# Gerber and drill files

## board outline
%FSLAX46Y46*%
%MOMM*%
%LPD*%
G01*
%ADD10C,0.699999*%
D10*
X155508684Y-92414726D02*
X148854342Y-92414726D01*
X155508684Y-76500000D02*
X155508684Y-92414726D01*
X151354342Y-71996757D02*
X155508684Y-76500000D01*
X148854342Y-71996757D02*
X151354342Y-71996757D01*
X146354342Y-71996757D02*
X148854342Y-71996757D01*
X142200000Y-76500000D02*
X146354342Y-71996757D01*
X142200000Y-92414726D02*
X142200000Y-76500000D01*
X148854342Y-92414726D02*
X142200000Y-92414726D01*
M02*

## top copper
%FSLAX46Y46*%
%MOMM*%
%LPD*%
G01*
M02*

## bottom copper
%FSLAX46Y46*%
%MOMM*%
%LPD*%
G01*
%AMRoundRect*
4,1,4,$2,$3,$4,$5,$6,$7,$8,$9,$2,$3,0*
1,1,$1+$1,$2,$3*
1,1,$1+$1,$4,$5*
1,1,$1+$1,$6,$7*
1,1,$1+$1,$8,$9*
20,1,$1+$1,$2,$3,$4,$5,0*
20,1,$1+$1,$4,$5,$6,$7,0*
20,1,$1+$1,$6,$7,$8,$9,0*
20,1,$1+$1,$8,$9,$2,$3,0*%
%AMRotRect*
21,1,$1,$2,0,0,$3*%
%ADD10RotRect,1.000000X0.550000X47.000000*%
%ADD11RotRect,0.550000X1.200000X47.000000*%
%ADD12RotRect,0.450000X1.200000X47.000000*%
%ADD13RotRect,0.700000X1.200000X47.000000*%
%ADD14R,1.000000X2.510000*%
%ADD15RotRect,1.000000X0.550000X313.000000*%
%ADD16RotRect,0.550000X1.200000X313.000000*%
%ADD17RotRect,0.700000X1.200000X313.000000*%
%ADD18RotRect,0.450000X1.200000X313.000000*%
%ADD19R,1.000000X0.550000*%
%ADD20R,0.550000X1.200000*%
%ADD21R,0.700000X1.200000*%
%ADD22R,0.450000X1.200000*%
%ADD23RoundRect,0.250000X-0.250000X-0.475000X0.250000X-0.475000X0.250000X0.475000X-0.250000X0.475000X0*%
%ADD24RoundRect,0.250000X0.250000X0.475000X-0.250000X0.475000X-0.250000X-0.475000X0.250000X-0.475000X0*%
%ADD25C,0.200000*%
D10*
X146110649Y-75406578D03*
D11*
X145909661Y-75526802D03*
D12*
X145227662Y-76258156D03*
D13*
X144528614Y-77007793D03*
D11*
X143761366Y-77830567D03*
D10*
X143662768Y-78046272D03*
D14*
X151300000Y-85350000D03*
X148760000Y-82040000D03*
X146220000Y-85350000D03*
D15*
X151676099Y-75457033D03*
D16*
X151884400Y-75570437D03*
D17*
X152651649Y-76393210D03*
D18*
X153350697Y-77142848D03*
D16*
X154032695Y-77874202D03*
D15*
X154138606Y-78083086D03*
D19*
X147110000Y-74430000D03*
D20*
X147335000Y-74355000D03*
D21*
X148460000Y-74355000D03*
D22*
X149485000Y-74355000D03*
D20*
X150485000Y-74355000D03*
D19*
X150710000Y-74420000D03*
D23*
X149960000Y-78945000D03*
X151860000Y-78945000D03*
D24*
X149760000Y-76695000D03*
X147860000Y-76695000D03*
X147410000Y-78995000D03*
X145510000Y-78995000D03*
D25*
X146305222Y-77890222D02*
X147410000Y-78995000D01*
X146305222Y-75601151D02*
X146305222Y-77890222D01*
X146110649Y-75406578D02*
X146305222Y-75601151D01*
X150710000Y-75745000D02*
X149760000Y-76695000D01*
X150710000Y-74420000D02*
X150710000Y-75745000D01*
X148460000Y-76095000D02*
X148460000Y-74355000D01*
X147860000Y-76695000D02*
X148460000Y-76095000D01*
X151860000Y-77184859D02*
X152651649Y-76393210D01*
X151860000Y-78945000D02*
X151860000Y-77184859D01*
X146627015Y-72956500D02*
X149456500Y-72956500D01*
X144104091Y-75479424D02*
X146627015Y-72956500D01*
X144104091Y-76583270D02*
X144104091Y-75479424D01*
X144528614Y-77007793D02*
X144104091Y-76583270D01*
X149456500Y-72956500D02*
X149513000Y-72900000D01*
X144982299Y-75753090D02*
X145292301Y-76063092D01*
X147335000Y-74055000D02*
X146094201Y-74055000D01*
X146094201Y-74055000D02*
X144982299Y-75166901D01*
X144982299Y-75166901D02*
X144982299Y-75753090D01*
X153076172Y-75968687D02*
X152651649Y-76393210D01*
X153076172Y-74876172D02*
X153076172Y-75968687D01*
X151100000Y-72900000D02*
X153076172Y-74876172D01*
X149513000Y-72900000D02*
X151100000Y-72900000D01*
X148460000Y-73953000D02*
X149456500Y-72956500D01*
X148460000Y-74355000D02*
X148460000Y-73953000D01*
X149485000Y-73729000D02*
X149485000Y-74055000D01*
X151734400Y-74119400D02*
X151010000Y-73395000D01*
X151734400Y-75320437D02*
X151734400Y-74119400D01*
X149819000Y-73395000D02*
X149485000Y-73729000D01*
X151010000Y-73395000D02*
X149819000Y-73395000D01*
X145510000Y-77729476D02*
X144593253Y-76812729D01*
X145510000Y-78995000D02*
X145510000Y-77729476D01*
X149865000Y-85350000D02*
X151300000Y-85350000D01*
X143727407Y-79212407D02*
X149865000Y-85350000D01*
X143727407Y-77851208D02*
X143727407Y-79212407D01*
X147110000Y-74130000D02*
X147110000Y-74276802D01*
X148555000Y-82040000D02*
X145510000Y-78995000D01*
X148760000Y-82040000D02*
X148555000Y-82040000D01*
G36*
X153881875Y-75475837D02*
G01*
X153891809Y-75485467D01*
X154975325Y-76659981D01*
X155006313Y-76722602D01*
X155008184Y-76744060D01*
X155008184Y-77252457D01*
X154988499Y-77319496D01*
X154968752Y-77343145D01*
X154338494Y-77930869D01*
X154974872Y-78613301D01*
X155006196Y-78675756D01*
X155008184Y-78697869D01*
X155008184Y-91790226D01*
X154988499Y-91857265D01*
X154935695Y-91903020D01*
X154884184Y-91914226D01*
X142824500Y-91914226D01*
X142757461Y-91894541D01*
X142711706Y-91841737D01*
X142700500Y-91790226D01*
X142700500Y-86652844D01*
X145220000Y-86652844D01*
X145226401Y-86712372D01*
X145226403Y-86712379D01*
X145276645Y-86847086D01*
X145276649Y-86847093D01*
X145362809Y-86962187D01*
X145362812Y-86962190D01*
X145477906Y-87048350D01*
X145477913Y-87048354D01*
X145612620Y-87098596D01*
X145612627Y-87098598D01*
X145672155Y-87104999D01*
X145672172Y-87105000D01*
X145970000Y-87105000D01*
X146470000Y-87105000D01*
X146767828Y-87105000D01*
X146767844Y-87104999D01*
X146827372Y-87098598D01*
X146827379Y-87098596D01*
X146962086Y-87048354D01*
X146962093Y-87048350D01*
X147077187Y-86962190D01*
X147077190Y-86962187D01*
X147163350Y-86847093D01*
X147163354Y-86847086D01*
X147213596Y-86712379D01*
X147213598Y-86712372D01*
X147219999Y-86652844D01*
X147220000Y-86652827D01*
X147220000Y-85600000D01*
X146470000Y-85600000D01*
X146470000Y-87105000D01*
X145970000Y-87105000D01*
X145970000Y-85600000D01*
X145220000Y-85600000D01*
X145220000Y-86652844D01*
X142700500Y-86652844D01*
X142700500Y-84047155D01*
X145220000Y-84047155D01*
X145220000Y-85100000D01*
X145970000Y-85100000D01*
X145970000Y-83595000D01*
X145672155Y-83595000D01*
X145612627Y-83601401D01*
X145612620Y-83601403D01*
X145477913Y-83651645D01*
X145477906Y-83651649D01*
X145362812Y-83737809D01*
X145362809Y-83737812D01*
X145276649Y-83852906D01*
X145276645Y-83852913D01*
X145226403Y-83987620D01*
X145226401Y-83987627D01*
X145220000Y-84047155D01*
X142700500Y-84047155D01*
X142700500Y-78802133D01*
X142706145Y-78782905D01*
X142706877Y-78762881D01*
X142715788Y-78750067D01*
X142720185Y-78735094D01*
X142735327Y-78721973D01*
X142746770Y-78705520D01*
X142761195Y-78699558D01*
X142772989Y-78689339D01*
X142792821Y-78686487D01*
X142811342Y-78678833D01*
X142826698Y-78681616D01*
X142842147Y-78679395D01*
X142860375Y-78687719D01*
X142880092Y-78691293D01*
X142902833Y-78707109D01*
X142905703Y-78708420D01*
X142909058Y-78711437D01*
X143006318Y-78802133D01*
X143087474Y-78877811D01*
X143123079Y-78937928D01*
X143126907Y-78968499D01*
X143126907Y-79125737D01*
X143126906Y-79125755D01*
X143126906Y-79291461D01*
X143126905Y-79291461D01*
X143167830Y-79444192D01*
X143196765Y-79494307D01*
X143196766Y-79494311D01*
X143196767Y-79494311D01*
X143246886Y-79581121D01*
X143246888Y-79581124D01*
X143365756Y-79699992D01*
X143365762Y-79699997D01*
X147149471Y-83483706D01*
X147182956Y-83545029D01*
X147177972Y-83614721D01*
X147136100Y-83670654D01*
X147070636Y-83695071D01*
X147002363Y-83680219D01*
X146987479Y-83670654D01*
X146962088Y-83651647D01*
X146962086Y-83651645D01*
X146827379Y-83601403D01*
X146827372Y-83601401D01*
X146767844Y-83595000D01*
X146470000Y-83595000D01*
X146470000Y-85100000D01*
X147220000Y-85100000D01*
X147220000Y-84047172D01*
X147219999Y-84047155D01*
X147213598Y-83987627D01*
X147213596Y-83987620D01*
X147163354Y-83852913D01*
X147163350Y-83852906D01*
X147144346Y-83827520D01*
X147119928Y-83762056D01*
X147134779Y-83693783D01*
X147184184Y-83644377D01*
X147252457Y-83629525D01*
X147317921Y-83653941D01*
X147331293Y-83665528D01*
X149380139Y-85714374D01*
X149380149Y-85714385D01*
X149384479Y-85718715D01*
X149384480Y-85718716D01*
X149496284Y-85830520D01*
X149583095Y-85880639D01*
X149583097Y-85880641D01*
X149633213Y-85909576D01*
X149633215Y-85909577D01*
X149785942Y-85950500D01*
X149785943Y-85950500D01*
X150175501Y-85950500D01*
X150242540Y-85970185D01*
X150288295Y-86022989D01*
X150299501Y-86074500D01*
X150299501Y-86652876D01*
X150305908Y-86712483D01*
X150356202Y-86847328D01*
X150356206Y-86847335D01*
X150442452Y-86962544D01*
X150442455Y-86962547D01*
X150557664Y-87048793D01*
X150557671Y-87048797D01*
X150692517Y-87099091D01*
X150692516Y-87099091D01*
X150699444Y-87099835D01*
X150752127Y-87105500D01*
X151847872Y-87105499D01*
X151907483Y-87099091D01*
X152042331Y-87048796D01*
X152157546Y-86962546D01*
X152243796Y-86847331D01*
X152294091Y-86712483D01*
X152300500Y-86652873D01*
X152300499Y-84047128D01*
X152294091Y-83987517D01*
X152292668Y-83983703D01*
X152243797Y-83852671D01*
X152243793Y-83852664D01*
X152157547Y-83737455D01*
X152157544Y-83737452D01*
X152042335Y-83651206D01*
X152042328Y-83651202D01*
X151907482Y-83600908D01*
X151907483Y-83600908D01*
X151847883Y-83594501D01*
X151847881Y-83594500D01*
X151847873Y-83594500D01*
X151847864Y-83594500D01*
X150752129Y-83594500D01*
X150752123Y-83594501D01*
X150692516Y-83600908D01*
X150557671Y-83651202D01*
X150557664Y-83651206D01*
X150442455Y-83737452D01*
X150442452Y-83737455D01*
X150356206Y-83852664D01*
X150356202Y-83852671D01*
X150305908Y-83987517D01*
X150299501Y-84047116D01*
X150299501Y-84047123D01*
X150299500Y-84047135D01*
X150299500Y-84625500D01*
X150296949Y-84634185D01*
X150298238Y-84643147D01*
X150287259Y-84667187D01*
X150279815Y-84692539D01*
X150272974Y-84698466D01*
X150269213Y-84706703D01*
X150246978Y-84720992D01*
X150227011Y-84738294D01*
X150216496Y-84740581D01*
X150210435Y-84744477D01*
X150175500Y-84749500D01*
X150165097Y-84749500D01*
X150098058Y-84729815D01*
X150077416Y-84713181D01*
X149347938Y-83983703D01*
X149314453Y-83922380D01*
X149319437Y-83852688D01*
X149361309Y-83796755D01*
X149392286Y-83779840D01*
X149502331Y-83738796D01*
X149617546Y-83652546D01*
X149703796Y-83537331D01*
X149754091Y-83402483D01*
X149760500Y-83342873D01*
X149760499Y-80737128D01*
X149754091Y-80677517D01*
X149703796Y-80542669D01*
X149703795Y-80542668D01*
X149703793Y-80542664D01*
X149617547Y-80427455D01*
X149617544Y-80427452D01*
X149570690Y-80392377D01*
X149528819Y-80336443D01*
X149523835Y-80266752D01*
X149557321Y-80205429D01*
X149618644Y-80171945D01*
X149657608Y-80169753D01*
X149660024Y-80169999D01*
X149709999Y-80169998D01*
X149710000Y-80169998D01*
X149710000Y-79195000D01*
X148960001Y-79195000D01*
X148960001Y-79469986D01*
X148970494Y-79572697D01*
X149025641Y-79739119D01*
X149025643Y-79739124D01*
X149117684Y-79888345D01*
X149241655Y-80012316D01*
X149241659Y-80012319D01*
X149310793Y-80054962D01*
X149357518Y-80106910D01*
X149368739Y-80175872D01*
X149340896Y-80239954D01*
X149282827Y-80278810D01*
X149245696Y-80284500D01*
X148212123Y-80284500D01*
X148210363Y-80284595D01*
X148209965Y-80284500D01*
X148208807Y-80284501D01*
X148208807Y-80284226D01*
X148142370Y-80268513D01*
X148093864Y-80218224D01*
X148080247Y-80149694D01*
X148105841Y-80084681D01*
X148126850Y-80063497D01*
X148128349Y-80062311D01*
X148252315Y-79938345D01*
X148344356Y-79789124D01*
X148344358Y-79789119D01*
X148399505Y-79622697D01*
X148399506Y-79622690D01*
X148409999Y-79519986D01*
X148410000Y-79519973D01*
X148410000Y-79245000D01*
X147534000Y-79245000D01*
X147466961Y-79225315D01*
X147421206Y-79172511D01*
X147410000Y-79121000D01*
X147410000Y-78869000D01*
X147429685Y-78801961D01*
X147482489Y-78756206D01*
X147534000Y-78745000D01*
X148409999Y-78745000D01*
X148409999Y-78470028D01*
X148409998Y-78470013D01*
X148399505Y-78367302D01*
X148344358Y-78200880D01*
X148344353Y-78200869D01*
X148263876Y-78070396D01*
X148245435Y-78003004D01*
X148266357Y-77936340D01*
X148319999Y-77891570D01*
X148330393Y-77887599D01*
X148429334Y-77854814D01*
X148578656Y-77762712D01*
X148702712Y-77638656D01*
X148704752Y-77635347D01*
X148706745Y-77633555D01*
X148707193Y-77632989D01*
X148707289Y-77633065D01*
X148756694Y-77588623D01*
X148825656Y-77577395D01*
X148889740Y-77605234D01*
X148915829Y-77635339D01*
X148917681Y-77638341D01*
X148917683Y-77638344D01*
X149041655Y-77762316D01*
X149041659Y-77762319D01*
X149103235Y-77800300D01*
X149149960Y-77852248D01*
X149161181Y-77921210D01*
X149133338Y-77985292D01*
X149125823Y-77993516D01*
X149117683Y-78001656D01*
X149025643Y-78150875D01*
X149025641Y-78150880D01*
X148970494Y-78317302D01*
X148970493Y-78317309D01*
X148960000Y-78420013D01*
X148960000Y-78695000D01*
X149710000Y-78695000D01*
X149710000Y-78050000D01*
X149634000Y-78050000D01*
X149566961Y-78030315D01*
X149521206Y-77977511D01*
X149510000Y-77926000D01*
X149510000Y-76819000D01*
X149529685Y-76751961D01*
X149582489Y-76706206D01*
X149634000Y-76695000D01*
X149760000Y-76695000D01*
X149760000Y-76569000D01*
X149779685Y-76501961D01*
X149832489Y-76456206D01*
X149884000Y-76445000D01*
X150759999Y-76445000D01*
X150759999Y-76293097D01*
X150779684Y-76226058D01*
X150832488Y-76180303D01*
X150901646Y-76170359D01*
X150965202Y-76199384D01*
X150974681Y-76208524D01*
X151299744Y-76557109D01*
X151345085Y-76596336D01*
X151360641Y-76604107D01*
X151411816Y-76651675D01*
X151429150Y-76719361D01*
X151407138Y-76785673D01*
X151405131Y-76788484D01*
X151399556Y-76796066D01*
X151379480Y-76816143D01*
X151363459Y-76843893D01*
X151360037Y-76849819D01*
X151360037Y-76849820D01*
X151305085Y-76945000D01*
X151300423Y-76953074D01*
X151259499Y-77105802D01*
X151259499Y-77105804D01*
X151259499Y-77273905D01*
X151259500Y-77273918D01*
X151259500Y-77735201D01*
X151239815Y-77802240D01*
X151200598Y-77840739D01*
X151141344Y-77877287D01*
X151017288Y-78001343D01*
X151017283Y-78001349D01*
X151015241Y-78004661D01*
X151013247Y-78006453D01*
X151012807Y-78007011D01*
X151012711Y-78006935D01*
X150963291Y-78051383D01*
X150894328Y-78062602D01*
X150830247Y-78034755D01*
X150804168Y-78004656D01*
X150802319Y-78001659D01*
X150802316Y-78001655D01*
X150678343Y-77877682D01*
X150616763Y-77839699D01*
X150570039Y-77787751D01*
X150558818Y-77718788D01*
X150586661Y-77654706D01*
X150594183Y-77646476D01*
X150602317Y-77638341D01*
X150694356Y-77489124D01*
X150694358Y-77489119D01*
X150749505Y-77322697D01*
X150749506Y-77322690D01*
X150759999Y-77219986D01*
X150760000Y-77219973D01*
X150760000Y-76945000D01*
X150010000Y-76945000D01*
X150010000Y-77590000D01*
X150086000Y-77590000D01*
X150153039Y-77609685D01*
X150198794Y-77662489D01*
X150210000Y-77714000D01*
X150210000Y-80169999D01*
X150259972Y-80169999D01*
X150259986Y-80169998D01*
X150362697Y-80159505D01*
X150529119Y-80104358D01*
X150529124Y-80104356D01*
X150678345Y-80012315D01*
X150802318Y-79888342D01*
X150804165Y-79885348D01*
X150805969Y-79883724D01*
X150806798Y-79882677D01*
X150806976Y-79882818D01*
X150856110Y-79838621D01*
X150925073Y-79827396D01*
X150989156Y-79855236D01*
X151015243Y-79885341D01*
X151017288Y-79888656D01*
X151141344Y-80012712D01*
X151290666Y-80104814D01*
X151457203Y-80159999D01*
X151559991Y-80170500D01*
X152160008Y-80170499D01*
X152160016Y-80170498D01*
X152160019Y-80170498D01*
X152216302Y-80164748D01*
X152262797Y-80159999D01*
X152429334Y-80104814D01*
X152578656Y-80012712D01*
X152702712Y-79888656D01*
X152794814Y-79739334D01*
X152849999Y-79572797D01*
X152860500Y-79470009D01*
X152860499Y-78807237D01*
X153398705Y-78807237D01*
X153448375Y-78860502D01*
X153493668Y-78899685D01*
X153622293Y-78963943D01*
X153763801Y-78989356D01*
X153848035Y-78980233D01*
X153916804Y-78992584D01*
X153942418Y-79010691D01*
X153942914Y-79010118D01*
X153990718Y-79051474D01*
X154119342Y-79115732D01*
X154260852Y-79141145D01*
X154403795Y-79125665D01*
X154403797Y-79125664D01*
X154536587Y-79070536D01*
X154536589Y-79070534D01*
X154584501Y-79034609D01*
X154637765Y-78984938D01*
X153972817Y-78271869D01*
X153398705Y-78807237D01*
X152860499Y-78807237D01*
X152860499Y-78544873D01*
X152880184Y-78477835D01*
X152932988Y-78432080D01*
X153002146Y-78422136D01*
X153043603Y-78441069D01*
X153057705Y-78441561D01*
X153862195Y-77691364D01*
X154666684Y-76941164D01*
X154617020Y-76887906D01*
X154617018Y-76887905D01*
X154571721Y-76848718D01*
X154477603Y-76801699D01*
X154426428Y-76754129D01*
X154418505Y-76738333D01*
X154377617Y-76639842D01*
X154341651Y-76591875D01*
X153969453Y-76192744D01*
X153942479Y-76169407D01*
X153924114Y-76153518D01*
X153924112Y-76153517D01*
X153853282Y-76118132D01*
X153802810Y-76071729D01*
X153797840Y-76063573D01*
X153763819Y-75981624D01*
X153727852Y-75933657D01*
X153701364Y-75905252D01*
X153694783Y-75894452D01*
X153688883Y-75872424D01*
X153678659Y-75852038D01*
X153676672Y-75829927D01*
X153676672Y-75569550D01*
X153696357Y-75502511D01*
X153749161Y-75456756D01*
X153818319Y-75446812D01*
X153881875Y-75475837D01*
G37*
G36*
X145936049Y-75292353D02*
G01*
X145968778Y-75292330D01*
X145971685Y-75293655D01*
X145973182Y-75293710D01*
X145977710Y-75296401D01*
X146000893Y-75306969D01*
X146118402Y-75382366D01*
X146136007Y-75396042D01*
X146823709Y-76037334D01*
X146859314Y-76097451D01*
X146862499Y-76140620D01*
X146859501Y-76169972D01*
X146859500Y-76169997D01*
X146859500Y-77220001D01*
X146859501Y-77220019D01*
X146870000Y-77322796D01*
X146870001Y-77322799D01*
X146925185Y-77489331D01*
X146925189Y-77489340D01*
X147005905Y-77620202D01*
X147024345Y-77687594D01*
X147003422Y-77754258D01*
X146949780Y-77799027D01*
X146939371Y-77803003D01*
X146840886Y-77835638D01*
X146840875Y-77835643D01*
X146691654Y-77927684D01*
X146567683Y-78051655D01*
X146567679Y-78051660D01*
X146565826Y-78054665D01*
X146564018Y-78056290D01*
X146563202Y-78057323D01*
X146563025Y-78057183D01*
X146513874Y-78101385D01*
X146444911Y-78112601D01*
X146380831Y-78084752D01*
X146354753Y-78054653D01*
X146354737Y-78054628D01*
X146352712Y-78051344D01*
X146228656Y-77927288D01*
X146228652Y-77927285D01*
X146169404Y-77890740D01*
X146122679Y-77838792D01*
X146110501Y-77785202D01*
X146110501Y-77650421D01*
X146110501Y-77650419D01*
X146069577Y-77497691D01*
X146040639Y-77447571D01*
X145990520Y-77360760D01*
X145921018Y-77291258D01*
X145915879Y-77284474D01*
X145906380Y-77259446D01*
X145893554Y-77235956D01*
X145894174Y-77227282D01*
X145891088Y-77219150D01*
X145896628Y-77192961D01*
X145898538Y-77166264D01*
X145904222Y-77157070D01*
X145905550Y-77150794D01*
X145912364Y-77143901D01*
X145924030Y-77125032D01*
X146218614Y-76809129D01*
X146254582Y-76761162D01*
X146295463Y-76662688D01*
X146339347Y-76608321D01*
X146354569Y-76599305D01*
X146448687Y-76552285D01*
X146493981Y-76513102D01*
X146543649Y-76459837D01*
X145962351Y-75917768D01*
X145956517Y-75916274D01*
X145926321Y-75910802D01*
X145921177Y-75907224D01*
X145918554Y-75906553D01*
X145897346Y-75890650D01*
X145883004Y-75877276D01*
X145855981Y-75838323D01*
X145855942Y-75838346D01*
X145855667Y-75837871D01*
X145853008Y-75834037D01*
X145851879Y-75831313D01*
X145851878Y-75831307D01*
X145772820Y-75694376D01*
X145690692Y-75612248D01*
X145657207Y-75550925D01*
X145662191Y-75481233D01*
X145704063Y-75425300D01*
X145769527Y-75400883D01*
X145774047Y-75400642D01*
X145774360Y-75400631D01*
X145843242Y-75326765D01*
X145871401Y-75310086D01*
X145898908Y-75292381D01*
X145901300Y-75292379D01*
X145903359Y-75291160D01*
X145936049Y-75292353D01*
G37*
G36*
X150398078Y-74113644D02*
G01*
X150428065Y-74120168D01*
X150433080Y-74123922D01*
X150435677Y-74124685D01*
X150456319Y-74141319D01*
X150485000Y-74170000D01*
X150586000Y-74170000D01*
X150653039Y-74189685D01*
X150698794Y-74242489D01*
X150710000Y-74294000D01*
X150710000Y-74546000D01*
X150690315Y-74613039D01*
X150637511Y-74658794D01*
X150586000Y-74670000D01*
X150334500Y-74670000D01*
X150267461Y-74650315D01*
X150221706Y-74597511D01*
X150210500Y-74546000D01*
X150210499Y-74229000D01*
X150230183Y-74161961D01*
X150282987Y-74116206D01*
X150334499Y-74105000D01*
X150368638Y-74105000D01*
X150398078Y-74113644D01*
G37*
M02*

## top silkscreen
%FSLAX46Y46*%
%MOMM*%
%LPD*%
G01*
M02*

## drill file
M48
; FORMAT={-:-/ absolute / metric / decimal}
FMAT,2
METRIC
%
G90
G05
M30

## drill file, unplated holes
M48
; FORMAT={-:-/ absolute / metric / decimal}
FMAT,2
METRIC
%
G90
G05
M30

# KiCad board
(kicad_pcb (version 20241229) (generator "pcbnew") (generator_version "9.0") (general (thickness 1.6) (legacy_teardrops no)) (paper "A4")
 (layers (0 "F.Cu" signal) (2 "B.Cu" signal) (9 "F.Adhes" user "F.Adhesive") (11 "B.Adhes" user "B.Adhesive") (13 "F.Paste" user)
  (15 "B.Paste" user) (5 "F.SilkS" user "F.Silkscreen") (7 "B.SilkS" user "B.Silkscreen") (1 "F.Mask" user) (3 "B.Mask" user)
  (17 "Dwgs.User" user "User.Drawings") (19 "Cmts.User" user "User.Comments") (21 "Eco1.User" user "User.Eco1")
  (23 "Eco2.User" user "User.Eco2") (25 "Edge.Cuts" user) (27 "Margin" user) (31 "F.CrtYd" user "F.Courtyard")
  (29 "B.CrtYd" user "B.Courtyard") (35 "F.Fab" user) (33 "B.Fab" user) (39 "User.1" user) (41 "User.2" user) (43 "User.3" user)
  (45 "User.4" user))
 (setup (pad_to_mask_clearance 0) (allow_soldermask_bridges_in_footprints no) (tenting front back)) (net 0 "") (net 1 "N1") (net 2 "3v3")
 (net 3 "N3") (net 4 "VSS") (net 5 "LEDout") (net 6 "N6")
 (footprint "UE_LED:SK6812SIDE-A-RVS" (layer "B.Cu") (at 152.897661 76.642364 -47)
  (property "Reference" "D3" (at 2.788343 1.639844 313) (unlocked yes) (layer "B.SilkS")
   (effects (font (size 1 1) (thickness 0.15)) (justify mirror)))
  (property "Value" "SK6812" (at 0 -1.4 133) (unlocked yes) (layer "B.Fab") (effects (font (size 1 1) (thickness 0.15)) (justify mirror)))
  (pad "1" smd rect (at -1.699999 0.085 313) (size 1 0.55) (layers "B.Cu" "B.Mask" "B.Paste") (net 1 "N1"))
  (pad "1" smd rect (at -1.475 0.01 313) (size 0.55 1.2) (layers "B.Cu" "B.Mask" "B.Paste") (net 1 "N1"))
  (pad "2" smd rect (at -0.349999 0.009999 313) (size 0.7 1.2) (layers "B.Cu" "B.Mask" "B.Paste") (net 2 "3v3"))
  (pad "3" smd rect (at 0.675001 0.01 313) (size 0.45 1.2) (layers "B.Cu" "B.Mask" "B.Paste") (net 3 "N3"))
  (pad "4" smd rect (at 1.675001 0.01 313) (size 0.55 1.2) (layers "B.Cu" "B.Mask" "B.Paste") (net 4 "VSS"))
  (pad "4" smd rect (at 1.9 0.075 313) (size 1 0.55) (layers "B.Cu" "B.Mask" "B.Paste") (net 4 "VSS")))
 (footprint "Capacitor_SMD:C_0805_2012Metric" (layer "B.Cu") (at 150.91 78.945)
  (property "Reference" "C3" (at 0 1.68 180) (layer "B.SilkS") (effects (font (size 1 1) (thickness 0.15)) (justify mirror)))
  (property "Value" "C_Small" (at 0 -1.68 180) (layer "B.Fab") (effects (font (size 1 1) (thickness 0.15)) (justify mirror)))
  (pad "1" smd roundrect (at -0.95 0) (size 1 1.45) (layers "B.Cu" "B.Mask" "B.Paste") (roundrect_rratio 0.25) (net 4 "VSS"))
  (pad "2" smd roundrect (at 0.95 0) (size 1 1.45) (layers "B.Cu" "B.Mask" "B.Paste") (roundrect_rratio 0.25) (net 2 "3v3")))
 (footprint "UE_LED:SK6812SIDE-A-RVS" (layer "B.Cu") (at 144.76 76.745 47)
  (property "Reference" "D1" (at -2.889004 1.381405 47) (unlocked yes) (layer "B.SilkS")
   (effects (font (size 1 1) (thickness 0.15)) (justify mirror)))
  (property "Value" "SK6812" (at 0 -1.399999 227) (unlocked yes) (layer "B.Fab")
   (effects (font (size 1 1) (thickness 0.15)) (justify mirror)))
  (pad "1" smd rect (at -1.700001 0.085001 47) (size 1 0.55) (layers "B.Cu" "B.Mask" "B.Paste") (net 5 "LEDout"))
  (pad "1" smd rect (at -1.475 0.01 47) (size 0.55 1.2) (layers "B.Cu" "B.Mask" "B.Paste") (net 5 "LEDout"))
  (pad "2" smd rect (at -0.35 0.009999 47) (size 0.7 1.2) (layers "B.Cu" "B.Mask" "B.Paste") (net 2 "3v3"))
  (pad "3" smd rect (at 0.675 0.01 47) (size 0.45 1.2) (layers "B.Cu" "B.Mask" "B.Paste") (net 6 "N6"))
  (pad "4" smd rect (at 1.675001 0.01 47) (size 0.55 1.2) (layers "B.Cu" "B.Mask" "B.Paste") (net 4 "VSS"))
  (pad "4" smd rect (at 1.9 0.075001 47) (size 1 0.55) (layers "B.Cu" "B.Mask" "B.Paste") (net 4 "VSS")))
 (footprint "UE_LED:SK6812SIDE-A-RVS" (layer "B.Cu") (at 148.81 74.345)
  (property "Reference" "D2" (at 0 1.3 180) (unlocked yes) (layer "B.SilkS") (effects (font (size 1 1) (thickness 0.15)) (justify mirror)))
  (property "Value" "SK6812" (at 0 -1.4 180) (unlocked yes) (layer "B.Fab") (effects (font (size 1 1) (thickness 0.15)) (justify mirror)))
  (pad "1" smd rect (at -1.7 0.085) (size 1 0.55) (layers "B.Cu" "B.Mask" "B.Paste") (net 6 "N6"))
  (pad "1" smd rect (at -1.475 0.01) (size 0.55 1.2) (layers "B.Cu" "B.Mask" "B.Paste") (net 6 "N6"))
  (pad "2" smd rect (at -0.35 0.01) (size 0.7 1.2) (layers "B.Cu" "B.Mask" "B.Paste") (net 2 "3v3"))
  (pad "3" smd rect (at 0.675 0.01) (size 0.45 1.2) (layers "B.Cu" "B.Mask" "B.Paste") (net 1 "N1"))
  (pad "4" smd rect (at 1.675 0.01) (size 0.55 1.2) (layers "B.Cu" "B.Mask" "B.Paste") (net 4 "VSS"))
  (pad "4" smd rect (at 1.9 0.075) (size 1 0.55) (layers "B.Cu" "B.Mask" "B.Paste") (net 4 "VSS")))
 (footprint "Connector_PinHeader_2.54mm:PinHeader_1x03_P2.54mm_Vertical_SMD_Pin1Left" (layer "B.Cu") (at 148.76 83.695 90)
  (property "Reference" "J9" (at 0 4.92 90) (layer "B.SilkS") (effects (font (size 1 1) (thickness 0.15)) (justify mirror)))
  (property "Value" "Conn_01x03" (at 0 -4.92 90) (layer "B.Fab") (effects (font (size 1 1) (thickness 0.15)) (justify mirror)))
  (pad "1" smd rect (at -1.655 2.54 90) (size 2.51 1) (layers "B.Cu" "B.Mask" "B.Paste") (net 5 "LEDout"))
  (pad "2" smd rect (at 1.655 0 90) (size 2.51 1) (layers "B.Cu" "B.Mask" "B.Paste") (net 2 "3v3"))
  (pad "3" smd rect (at -1.655 -2.54 90) (size 2.51 1) (layers "B.Cu" "B.Mask" "B.Paste") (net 4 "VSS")))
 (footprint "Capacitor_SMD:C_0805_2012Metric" (layer "B.Cu") (at 148.81 76.695 180)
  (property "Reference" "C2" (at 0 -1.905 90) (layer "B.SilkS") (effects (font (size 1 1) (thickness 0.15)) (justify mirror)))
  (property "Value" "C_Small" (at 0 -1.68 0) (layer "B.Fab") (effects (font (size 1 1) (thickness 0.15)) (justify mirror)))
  (pad "1" smd roundrect (at -0.95 0 180) (size 1 1.45) (layers "B.Cu" "B.Mask" "B.Paste") (roundrect_rratio 0.25) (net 4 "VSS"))
  (pad "2" smd roundrect (at 0.95 0 180) (size 1 1.45) (layers "B.Cu" "B.Mask" "B.Paste") (roundrect_rratio 0.25) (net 2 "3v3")))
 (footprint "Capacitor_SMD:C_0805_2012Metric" (layer "B.Cu") (at 146.46 78.995 180)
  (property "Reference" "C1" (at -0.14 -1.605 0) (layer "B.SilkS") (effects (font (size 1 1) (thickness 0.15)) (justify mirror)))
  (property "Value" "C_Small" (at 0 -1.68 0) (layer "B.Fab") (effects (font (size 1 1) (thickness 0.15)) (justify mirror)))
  (pad "1" smd roundrect (at -0.95 0 180) (size 1 1.45) (layers "B.Cu" "B.Mask" "B.Paste") (roundrect_rratio 0.25) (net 4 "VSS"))
  (pad "2" smd roundrect (at 0.95 0 180) (size 1 1.45) (layers "B.Cu" "B.Mask" "B.Paste") (roundrect_rratio 0.25) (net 2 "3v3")))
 (gr_line (start 142.2 76.5) (end 146.354342 71.996757) (stroke (width 0.699999) (type solid) (color 33 37 41 1)) (layer "Edge.Cuts"))
 (gr_line (start 151.354342 71.996757) (end 155.508684 76.5) (stroke (width 0.699999) (type solid) (color 33 37 41 1)) (layer "Edge.Cuts"))
 (gr_line (start 155.508684 92.414726) (end 148.854342 92.414726) (stroke (width 0.699999) (type solid) (color 33 37 41 1))
  (layer "Edge.Cuts"))
 (gr_line (start 142.2 92.414726) (end 142.2 76.5) (stroke (width 0.699999) (type solid) (color 33 37 41 1)) (layer "Edge.Cuts"))
 (gr_line (start 148.854342 92.414726) (end 142.2 92.414726) (stroke (width 0.699999) (type solid) (color 33 37 41 1)) (layer "Edge.Cuts"))
 (gr_line (start 146.354342 71.996757) (end 148.854342 71.996757) (stroke (width 0.699999) (type solid) (color 33 37 41 1))
  (layer "Edge.Cuts"))
 (gr_line (start 148.854342 71.996757) (end 151.354342 71.996757) (stroke (width 0.699999) (type solid) (color 33 37 41 1))
  (layer "Edge.Cuts"))
 (gr_line (start 155.508684 76.5) (end 155.508684 92.414726) (stroke (width 0.699999) (type solid) (color 33 37 41 1)) (layer "Edge.Cuts"))
 (segment (start 151.86 78.945) (end 151.86 77.184859) (width 0.2) (layer "B.Cu") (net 2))
 (segment (start 148.76 82.04) (end 148.555 82.04) (width 0.2) (layer "B.Cu") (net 2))
 (segment (start 146.627015 72.9565) (end 149.4565 72.9565) (width 0.2) (layer "B.Cu") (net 2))
 (segment (start 144.104091 75.479424) (end 146.627015 72.9565) (width 0.2) (layer "B.Cu") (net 2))
 (segment (start 145.51 78.995) (end 145.51 77.729476) (width 0.2) (layer "B.Cu") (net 2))
 (segment (start 148.46 73.953) (end 149.4565 72.9565) (width 0.2) (layer "B.Cu") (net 2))
 (segment (start 148.46 76.095) (end 148.46 74.355) (width 0.2) (layer "B.Cu") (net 2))
 (segment (start 147.86 76.695) (end 148.46 76.095) (width 0.2) (layer "B.Cu") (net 2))
 (segment (start 145.51 77.729476) (end 144.593253 76.812729) (width 0.2) (layer "B.Cu") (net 2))
 (segment (start 153.076172 74.876172) (end 153.076172 75.968687) (width 0.2) (layer "B.Cu") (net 2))
 (segment (start 148.46 74.355) (end 148.46 73.953) (width 0.2) (layer "B.Cu") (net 2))
 (segment (start 148.555 82.04) (end 145.51 78.995) (width 0.2) (layer "B.Cu") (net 2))
 (segment (start 151.1 72.9) (end 153.076172 74.876172) (width 0.2) (layer "B.Cu") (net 2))
 (segment (start 149.513 72.9) (end 151.1 72.9) (width 0.2) (layer "B.Cu") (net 2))
 (segment (start 151.86 77.184859) (end 152.651649 76.39321) (width 0.2) (layer "B.Cu") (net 2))
 (segment (start 144.104091 76.58327) (end 144.104091 75.479424) (width 0.2) (layer "B.Cu") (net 2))
 (segment (start 153.076172 75.968687) (end 152.651649 76.39321) (width 0.2) (layer "B.Cu") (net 2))
 (segment (start 144.528614 77.007793) (end 144.104091 76.58327) (width 0.2) (layer "B.Cu") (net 2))
 (segment (start 149.4565 72.9565) (end 149.513 72.9) (width 0.2) (layer "B.Cu") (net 2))
 (segment (start 146.110649 75.406578) (end 146.305222 75.601151) (width 0.2) (layer "B.Cu") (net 4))
 (segment (start 150.71 75.745) (end 149.76 76.695) (width 0.2) (layer "B.Cu") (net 4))
 (segment (start 146.305222 77.890222) (end 147.41 78.995) (width 0.2) (layer "B.Cu") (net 4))
 (segment (start 150.71 74.42) (end 150.71 75.745) (width 0.2) (layer "B.Cu") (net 4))
 (segment (start 146.305222 75.601151) (end 146.305222 77.890222) (width 0.2) (layer "B.Cu") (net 4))
 (segment (start 143.727407 77.851208) (end 143.727407 79.212407) (width 0.2) (layer "B.Cu") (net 5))
 (segment (start 149.865 85.35) (end 151.3 85.35) (width 0.2) (layer "B.Cu") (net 5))
 (segment (start 143.727407 79.212407) (end 149.865 85.35) (width 0.2) (layer "B.Cu") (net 5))
 (segment (start 144.982299 75.75309) (end 145.292301 76.063092) (width 0.2) (layer "B.Cu") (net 6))
 (segment (start 144.982299 75.166901) (end 144.982299 75.75309) (width 0.2) (layer "B.Cu") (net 6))
 (segment (start 147.335 74.055) (end 146.094201 74.055) (width 0.2) (layer "B.Cu") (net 6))
 (segment (start 147.11 74.13) (end 147.11 74.276802) (width 0.2) (layer "B.Cu") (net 6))
 (segment (start 146.094201 74.055) (end 144.982299 75.166901) (width 0.2) (layer "B.Cu") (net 6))
 (segment (start 151.7344 74.1194) (end 151.01 73.395) (width 0.2) (layer "B.Cu") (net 1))
 (segment (start 151.01 73.395) (end 149.819 73.395) (width 0.2) (layer "B.Cu") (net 1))
 (segment (start 149.485 73.729) (end 149.485 74.055) (width 0.2) (layer "B.Cu") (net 1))
 (segment (start 149.819 73.395) (end 149.485 73.729) (width 0.2) (layer "B.Cu") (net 1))
 (segment (start 151.7344 75.320437) (end 151.7344 74.1194) (width 0.2) (layer "B.Cu") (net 1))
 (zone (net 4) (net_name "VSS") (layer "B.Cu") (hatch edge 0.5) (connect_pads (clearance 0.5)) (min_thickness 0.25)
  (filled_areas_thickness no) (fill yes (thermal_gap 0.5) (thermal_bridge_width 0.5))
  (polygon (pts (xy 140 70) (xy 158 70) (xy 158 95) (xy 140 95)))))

